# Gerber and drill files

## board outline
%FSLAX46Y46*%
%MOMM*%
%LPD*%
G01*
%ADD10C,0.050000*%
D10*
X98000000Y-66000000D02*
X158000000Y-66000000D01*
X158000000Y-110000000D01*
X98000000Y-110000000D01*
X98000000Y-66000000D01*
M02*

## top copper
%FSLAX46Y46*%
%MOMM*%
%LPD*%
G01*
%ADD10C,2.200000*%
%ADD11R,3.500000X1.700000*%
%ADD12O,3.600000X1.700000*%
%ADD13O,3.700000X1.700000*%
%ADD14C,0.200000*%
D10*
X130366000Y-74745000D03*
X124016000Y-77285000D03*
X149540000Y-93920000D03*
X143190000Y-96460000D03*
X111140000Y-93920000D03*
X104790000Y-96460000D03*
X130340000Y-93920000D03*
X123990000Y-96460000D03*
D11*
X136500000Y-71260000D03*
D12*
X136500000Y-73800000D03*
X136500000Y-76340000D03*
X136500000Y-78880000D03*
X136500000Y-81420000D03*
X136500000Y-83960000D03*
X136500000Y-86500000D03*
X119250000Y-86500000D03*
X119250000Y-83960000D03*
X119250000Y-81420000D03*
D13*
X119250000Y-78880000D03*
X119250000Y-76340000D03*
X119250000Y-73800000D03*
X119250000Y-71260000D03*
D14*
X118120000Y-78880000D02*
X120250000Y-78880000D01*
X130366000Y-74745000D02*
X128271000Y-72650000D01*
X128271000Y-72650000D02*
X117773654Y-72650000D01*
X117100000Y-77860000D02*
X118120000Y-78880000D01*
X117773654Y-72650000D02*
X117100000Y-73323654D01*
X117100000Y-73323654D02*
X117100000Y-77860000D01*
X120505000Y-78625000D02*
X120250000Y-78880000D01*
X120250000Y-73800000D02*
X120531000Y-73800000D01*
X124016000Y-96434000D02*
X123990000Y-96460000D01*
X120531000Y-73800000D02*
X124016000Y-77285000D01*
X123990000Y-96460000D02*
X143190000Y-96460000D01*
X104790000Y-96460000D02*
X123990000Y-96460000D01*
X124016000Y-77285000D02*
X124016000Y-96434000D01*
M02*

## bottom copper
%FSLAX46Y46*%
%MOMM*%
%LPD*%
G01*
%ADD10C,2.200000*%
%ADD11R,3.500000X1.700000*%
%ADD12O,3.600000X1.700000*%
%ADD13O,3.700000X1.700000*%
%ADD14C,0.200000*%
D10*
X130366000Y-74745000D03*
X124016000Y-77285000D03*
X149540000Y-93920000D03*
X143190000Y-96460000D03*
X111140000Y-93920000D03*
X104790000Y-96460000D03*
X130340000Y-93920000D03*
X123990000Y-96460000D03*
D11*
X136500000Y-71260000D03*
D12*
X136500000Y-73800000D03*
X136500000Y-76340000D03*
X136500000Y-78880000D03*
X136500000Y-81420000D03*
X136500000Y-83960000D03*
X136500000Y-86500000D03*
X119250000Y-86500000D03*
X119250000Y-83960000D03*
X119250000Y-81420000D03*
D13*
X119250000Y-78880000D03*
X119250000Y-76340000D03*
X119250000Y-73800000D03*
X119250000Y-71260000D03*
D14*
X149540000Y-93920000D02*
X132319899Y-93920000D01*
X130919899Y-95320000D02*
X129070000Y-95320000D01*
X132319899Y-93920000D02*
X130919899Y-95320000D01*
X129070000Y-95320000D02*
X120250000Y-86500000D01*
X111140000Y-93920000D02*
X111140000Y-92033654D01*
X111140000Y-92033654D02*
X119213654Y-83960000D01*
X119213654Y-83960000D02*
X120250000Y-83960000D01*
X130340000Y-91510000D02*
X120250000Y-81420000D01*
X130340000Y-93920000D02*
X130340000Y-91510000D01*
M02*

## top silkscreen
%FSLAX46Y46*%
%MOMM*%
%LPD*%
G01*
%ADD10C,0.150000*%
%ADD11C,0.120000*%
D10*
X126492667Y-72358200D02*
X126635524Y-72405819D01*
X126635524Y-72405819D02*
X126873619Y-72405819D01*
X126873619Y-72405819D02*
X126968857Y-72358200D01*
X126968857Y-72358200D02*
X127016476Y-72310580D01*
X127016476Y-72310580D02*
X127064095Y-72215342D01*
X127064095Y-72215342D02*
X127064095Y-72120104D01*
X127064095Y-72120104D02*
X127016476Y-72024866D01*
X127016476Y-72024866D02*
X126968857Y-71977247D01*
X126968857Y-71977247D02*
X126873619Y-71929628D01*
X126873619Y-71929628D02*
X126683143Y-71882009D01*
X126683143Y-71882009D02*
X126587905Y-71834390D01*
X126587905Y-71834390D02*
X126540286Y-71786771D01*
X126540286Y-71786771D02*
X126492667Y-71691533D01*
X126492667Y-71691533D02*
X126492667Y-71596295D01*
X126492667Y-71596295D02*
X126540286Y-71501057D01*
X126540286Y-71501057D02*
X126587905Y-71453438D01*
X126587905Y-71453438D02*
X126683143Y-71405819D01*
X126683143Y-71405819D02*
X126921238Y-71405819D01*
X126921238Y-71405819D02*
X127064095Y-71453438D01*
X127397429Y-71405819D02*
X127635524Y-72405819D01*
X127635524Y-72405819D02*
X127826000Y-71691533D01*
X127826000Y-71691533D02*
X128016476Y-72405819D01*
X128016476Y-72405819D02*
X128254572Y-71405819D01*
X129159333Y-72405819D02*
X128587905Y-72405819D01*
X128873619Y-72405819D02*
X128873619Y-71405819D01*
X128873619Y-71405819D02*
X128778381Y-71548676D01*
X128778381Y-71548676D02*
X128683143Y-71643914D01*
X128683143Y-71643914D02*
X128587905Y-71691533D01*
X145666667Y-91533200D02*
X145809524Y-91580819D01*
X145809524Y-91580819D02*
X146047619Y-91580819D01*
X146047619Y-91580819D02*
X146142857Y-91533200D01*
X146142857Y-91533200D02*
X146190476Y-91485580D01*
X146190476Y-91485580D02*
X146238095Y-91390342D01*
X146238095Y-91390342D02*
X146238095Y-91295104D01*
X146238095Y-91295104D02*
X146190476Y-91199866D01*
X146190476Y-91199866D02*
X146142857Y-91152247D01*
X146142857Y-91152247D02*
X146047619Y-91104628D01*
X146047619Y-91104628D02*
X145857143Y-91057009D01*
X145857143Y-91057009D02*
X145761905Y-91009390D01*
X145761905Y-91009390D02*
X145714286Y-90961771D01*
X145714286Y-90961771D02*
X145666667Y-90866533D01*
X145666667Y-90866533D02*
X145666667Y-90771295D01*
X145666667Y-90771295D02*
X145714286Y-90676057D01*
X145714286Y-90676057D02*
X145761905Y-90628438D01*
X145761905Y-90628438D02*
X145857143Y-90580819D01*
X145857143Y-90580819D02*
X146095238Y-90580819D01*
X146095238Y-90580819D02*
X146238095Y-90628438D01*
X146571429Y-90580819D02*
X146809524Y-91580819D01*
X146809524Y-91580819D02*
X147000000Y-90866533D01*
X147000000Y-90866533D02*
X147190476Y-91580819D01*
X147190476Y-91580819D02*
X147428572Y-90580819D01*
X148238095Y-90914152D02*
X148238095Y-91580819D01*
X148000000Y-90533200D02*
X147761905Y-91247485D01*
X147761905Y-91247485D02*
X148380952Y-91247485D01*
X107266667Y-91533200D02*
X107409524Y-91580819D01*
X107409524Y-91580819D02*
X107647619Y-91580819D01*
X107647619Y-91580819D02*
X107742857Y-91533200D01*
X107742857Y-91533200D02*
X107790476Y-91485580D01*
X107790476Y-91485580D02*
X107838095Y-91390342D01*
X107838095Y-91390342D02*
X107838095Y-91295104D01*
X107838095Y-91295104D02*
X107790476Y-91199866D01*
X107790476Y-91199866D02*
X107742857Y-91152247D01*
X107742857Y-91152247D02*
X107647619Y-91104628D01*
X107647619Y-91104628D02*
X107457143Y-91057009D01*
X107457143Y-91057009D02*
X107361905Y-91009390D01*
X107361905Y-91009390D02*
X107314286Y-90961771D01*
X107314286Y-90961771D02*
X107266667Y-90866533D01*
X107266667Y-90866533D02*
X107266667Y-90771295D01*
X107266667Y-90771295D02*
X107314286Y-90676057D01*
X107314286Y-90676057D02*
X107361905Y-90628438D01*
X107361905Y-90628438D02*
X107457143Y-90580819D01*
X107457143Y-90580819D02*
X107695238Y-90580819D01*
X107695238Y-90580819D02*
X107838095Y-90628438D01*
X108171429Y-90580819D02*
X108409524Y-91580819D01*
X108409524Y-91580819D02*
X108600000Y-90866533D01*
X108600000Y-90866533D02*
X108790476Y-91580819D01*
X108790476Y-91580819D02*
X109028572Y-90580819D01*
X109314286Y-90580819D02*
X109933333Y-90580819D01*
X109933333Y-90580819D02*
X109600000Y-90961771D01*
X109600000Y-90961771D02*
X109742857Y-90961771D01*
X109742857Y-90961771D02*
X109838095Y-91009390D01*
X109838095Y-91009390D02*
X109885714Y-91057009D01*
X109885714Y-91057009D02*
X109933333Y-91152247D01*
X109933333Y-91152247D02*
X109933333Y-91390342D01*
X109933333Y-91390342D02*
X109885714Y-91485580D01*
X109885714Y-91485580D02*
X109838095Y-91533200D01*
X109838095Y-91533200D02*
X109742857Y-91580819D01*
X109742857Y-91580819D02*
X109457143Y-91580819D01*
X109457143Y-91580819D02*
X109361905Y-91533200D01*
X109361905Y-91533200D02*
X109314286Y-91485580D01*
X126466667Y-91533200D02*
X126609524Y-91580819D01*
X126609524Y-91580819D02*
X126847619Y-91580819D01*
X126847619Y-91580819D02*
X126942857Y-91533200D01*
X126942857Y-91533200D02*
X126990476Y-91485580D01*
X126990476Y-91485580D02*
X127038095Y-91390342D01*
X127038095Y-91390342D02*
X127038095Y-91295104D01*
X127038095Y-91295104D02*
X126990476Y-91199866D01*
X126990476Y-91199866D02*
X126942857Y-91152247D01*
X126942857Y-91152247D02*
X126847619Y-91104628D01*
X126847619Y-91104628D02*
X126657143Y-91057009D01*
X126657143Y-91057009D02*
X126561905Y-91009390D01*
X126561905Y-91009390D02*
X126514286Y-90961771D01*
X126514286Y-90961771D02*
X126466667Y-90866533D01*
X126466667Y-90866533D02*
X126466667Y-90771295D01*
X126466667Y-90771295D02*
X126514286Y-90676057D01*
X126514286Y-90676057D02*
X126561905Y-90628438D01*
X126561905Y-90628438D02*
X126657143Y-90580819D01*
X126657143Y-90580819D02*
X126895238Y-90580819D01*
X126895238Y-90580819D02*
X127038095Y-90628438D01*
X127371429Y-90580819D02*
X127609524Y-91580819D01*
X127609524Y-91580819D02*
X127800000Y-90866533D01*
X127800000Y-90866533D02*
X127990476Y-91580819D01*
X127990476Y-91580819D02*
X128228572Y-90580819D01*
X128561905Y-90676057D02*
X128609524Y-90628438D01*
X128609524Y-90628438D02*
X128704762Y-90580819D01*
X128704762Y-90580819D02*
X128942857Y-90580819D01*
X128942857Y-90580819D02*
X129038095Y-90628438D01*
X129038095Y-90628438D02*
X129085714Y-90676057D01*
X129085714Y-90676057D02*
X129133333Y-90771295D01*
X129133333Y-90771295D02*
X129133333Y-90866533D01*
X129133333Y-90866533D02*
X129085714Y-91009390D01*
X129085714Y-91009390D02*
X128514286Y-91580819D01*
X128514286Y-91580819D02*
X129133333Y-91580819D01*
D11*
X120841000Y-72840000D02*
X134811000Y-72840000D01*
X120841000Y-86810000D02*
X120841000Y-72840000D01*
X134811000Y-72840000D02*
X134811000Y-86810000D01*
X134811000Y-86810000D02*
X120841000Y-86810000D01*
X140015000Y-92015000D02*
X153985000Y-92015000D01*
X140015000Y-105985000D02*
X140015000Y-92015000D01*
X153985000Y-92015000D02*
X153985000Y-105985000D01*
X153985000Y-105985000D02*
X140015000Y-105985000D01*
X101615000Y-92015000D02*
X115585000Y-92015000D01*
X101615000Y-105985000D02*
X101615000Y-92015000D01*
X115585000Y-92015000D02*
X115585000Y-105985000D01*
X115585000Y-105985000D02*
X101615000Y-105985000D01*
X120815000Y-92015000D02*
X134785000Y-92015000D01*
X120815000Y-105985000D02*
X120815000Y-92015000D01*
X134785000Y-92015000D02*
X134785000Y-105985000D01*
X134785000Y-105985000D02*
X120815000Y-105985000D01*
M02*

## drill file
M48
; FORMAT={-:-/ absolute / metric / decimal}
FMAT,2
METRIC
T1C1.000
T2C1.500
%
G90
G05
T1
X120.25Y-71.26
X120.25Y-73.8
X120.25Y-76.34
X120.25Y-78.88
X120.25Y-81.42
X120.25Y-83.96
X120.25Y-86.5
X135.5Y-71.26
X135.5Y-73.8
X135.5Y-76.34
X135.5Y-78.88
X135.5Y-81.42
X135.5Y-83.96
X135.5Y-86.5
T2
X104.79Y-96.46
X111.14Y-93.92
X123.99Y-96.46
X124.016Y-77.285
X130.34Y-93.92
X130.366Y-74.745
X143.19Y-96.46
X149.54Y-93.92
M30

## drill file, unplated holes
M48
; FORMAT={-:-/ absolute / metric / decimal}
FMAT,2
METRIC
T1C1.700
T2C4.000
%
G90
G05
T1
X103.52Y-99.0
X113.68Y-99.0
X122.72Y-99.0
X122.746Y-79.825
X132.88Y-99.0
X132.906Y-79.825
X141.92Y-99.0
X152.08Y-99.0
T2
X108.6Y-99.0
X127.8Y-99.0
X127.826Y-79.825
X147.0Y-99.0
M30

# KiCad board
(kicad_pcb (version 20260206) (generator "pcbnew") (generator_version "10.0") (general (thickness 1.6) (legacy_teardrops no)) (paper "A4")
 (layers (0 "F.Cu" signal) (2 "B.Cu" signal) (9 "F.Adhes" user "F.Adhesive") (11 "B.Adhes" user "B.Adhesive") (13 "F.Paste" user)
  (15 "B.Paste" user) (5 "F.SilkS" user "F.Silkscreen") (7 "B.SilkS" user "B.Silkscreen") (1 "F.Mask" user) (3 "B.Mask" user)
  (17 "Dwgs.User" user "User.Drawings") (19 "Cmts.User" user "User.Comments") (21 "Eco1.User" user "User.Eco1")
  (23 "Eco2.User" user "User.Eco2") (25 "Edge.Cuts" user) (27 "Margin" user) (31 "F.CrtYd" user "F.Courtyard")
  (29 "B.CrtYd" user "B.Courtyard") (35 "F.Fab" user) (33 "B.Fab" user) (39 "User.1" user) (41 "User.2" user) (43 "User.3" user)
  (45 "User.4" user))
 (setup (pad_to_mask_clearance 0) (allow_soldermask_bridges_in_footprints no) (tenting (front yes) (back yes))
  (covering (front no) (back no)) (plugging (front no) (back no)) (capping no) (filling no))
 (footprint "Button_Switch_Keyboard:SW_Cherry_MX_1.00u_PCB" (layer "F.Cu") (at 130.366 74.745)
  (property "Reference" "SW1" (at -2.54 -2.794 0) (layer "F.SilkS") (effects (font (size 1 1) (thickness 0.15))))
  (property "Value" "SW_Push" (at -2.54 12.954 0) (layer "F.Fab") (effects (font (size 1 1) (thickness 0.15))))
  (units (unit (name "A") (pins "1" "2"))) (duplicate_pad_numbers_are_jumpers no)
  (fp_line (start -9.525 -1.905) (end 4.445 -1.905) (stroke (width 0.12) (type solid)) (layer "F.SilkS"))
  (fp_line (start -9.525 12.065) (end -9.525 -1.905) (stroke (width 0.12) (type solid)) (layer "F.SilkS"))
  (fp_line (start 4.445 -1.905) (end 4.445 12.065) (stroke (width 0.12) (type solid)) (layer "F.SilkS"))
  (fp_line (start 4.445 12.065) (end -9.525 12.065) (stroke (width 0.12) (type solid)) (layer "F.SilkS"))
  (pad "" np_thru_hole circle (at -7.62 5.08) (size 1.7 1.7) (drill 1.7) (layers "*.Cu" "*.Mask"))
  (pad "" np_thru_hole circle (at -2.54 5.08) (size 4 4) (drill 4) (layers "*.Cu" "*.Mask"))
  (pad "" np_thru_hole circle (at 2.54 5.08) (size 1.7 1.7) (drill 1.7) (layers "*.Cu" "*.Mask"))
  (pad "1" thru_hole circle (at 0 0) (size 2.2 2.2) (drill 1.5) (layers "*.Cu" "*.Mask") (remove_unused_layers no)
   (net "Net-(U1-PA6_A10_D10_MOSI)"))
  (pad "2" thru_hole circle (at -6.35 2.54) (size 2.2 2.2) (drill 1.5) (layers "*.Cu" "*.Mask") (remove_unused_layers no) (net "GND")))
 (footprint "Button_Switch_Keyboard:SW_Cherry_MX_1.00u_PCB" (layer "F.Cu") (at 149.54 93.92)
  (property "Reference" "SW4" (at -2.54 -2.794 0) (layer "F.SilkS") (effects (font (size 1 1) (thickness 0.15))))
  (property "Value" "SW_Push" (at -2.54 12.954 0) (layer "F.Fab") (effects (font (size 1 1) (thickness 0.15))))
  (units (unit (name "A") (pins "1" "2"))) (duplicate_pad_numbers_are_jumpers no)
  (fp_line (start -9.525 -1.905) (end 4.445 -1.905) (stroke (width 0.12) (type solid)) (layer "F.SilkS"))
  (fp_line (start -9.525 12.065) (end -9.525 -1.905) (stroke (width 0.12) (type solid)) (layer "F.SilkS"))
  (fp_line (start 4.445 -1.905) (end 4.445 12.065) (stroke (width 0.12) (type solid)) (layer "F.SilkS"))
  (fp_line (start 4.445 12.065) (end -9.525 12.065) (stroke (width 0.12) (type solid)) (layer "F.SilkS"))
  (pad "" np_thru_hole circle (at -7.62 5.08) (size 1.7 1.7) (drill 1.7) (layers "*.Cu" "*.Mask"))
  (pad "" np_thru_hole circle (at -2.54 5.08) (size 4 4) (drill 4) (layers "*.Cu" "*.Mask"))
  (pad "" np_thru_hole circle (at 2.54 5.08) (size 1.7 1.7) (drill 1.7) (layers "*.Cu" "*.Mask"))
  (pad "1" thru_hole circle (at 0 0) (size 2.2 2.2) (drill 1.5) (layers "*.Cu" "*.Mask") (remove_unused_layers no)
   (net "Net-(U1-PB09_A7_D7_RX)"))
  (pad "2" thru_hole circle (at -6.35 2.54) (size 2.2 2.2) (drill 1.5) (layers "*.Cu" "*.Mask") (remove_unused_layers no) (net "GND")))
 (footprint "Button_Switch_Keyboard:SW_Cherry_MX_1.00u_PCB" (layer "F.Cu") (at 111.14 93.92)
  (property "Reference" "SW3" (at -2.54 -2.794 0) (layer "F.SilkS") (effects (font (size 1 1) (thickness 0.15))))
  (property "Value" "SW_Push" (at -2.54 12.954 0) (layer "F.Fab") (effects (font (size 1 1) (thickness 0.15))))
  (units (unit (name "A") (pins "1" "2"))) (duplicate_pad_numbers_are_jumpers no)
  (fp_line (start -9.525 -1.905) (end 4.445 -1.905) (stroke (width 0.12) (type solid)) (layer "F.SilkS"))
  (fp_line (start -9.525 12.065) (end -9.525 -1.905) (stroke (width 0.12) (type solid)) (layer "F.SilkS"))
  (fp_line (start 4.445 -1.905) (end 4.445 12.065) (stroke (width 0.12) (type solid)) (layer "F.SilkS"))
  (fp_line (start 4.445 12.065) (end -9.525 12.065) (stroke (width 0.12) (type solid)) (layer "F.SilkS"))
  (pad "" np_thru_hole circle (at -7.62 5.08) (size 1.7 1.7) (drill 1.7) (layers "*.Cu" "*.Mask"))
  (pad "" np_thru_hole circle (at -2.54 5.08) (size 4 4) (drill 4) (layers "*.Cu" "*.Mask"))
  (pad "" np_thru_hole circle (at 2.54 5.08) (size 1.7 1.7) (drill 1.7) (layers "*.Cu" "*.Mask"))
  (pad "1" thru_hole circle (at 0 0) (size 2.2 2.2) (drill 1.5) (layers "*.Cu" "*.Mask") (remove_unused_layers no)
   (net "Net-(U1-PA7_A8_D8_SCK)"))
  (pad "2" thru_hole circle (at -6.35 2.54) (size 2.2 2.2) (drill 1.5) (layers "*.Cu" "*.Mask") (remove_unused_layers no) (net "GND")))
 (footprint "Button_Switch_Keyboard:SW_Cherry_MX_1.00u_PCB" (layer "F.Cu") (at 130.34 93.92)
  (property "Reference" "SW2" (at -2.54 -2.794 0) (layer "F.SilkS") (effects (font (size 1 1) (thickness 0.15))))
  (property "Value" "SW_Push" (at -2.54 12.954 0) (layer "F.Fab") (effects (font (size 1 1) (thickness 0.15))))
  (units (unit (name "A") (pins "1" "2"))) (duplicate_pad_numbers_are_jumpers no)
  (fp_line (start -9.525 -1.905) (end 4.445 -1.905) (stroke (width 0.12) (type solid)) (layer "F.SilkS"))
  (fp_line (start -9.525 12.065) (end -9.525 -1.905) (stroke (width 0.12) (type solid)) (layer "F.SilkS"))
  (fp_line (start 4.445 -1.905) (end 4.445 12.065) (stroke (width 0.12) (type solid)) (layer "F.SilkS"))
  (fp_line (start 4.445 12.065) (end -9.525 12.065) (stroke (width 0.12) (type solid)) (layer "F.SilkS"))
  (pad "" np_thru_hole circle (at -7.62 5.08) (size 1.7 1.7) (drill 1.7) (layers "*.Cu" "*.Mask"))
  (pad "" np_thru_hole circle (at -2.54 5.08) (size 4 4) (drill 4) (layers "*.Cu" "*.Mask"))
  (pad "" np_thru_hole circle (at 2.54 5.08) (size 1.7 1.7) (drill 1.7) (layers "*.Cu" "*.Mask"))
  (pad "1" thru_hole circle (at 0 0) (size 2.2 2.2) (drill 1.5) (layers "*.Cu" "*.Mask") (remove_unused_layers no)
   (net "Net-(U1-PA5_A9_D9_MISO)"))
  (pad "2" thru_hole circle (at -6.35 2.54) (size 2.2 2.2) (drill 1.5) (layers "*.Cu" "*.Mask") (remove_unused_layers no) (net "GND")))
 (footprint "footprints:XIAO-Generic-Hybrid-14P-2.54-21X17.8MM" (layer "B.Cu") (at 127.875 78.88 180)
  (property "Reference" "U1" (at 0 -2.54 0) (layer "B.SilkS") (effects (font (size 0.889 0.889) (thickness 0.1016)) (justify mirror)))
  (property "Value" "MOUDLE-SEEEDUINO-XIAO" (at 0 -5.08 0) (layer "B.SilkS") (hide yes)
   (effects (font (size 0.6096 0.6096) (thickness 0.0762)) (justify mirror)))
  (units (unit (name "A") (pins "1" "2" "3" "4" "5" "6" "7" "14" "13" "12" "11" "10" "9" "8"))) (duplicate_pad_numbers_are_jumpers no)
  (pad "1" thru_hole rect (at -7.625 7.62 180) (size 3.5 1.7) (drill 1 (offset -1 0)) (layers "*.Cu" "*.Mask") (remove_unused_layers no)
   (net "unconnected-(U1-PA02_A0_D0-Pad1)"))
  (pad "2" thru_hole oval (at -7.625 5.08 180) (size 3.6 1.7) (drill 1 (offset -1 0)) (layers "*.Cu" "*.Mask") (remove_unused_layers no)
   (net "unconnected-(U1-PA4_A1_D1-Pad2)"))
  (pad "3" thru_hole oval (at -7.625 2.54 180) (size 3.6 1.7) (drill 1 (offset -1 0)) (layers "*.Cu" "*.Mask") (remove_unused_layers no)
   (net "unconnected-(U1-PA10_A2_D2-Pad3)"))
  (pad "4" thru_hole oval (at -7.625 0 180) (size 3.6 1.7) (drill 1 (offset -1 0)) (layers "*.Cu" "*.Mask") (remove_unused_layers no)
   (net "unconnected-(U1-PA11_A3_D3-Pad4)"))
  (pad "5" thru_hole oval (at -7.625 -2.54 180) (size 3.6 1.7) (drill 1 (offset -1 0)) (layers "*.Cu" "*.Mask") (remove_unused_layers no)
   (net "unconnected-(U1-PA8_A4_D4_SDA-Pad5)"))
  (pad "6" thru_hole oval (at -7.625 -5.08) (size 3.6 1.7) (drill 1 (offset 1 0)) (layers "*.Cu" "*.Mask") (remove_unused_layers no)
   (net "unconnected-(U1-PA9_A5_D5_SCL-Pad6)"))
  (pad "7" thru_hole oval (at -7.625 -7.62 180) (size 3.6 1.7) (drill 1 (offset -1 0)) (layers "*.Cu" "*.Mask") (remove_unused_layers no)
   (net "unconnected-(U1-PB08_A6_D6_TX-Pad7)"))
  (pad "8" thru_hole oval (at 7.625 -7.62 180) (size 3.6 1.7) (drill 1 (offset 1 0)) (layers "*.Cu" "*.Mask") (remove_unused_layers no)
   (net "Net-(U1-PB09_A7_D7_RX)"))
  (pad "9" thru_hole oval (at 7.625 -5.08 180) (size 3.6 1.7) (drill 1 (offset 1 0)) (layers "*.Cu" "*.Mask") (remove_unused_layers no)
   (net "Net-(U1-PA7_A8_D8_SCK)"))
  (pad "10" thru_hole oval (at 7.625 -2.54 180) (size 3.6 1.7) (drill 1 (offset 1 0)) (layers "*.Cu" "*.Mask") (remove_unused_layers no)
   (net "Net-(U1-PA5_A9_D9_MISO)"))
  (pad "11" thru_hole oval (at 7.625 0 180) (size 3.7 1.7) (drill 1 (offset 1 0)) (layers "*.Cu" "*.Mask") (remove_unused_layers no)
   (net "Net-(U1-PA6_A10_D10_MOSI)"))
  (pad "12" thru_hole oval (at 7.625 2.54 180) (size 3.7 1.7) (drill 1 (offset 1 0)) (layers "*.Cu" "*.Mask") (remove_unused_layers no)
   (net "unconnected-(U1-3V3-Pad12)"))
  (pad "13" thru_hole oval (at 7.625 5.08 180) (size 3.7 1.7) (drill 1 (offset 1 0)) (layers "*.Cu" "*.Mask") (remove_unused_layers no)
   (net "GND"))
  (pad "14" thru_hole oval (at 7.625 7.62 180) (size 3.7 1.7) (drill 1 (offset 1 0)) (layers "*.Cu" "*.Mask") (remove_unused_layers no)
   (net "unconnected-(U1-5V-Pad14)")))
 (gr_rect (start 98 66) (end 158 110) (stroke (width 0.05) (type default)) (fill no) (layer "Edge.Cuts"))
 (segment (start 118.12 78.88) (end 120.25 78.88) (width 0.2) (layer "F.Cu") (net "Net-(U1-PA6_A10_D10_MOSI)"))
 (segment (start 130.366 74.745) (end 128.271 72.65) (width 0.2) (layer "F.Cu") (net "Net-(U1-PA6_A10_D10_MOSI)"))
 (segment (start 128.271 72.65) (end 117.773654 72.65) (width 0.2) (layer "F.Cu") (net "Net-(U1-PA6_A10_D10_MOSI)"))
 (segment (start 117.1 77.86) (end 118.12 78.88) (width 0.2) (layer "F.Cu") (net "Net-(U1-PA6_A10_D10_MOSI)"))
 (segment (start 117.773654 72.65) (end 117.1 73.323654) (width 0.2) (layer "F.Cu") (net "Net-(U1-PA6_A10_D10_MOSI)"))
 (segment (start 117.1 73.323654) (end 117.1 77.86) (width 0.2) (layer "F.Cu") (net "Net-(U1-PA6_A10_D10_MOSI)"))
 (segment (start 120.505 78.625) (end 120.25 78.88) (width 0.2) (layer "F.Cu") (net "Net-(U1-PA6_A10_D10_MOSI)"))
 (segment (start 120.25 73.8) (end 120.531 73.8) (width 0.2) (layer "F.Cu") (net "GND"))
 (segment (start 124.016 96.434) (end 123.99 96.46) (width 0.2) (layer "F.Cu") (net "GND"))
 (segment (start 120.531 73.8) (end 124.016 77.285) (width 0.2) (layer "F.Cu") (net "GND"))
 (segment (start 123.99 96.46) (end 143.19 96.46) (width 0.2) (layer "F.Cu") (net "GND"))
 (segment (start 104.79 96.46) (end 123.99 96.46) (width 0.2) (layer "F.Cu") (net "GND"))
 (segment (start 124.016 77.285) (end 124.016 96.434) (width 0.2) (layer "F.Cu") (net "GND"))
 (segment (start 149.54 93.92) (end 132.319899 93.92) (width 0.2) (layer "B.Cu") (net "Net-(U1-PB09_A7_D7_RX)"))
 (segment (start 130.919899 95.32) (end 129.07 95.32) (width 0.2) (layer "B.Cu") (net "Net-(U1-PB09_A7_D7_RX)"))
 (segment (start 132.319899 93.92) (end 130.919899 95.32) (width 0.2) (layer "B.Cu") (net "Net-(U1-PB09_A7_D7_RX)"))
 (segment (start 129.07 95.32) (end 120.25 86.5) (width 0.2) (layer "B.Cu") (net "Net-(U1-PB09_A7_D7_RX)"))
 (segment (start 111.14 93.92) (end 111.14 92.033654) (width 0.2) (layer "B.Cu") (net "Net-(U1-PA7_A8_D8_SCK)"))
 (segment (start 111.14 92.033654) (end 119.213654 83.96) (width 0.2) (layer "B.Cu") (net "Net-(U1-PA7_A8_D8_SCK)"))
 (segment (start 119.213654 83.96) (end 120.25 83.96) (width 0.2) (layer "B.Cu") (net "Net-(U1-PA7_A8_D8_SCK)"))
 (segment (start 130.34 91.51) (end 120.25 81.42) (width 0.2) (layer "B.Cu") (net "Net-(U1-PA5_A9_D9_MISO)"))
 (segment (start 130.34 93.92) (end 130.34 91.51) (width 0.2) (layer "B.Cu") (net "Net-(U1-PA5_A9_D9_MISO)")))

